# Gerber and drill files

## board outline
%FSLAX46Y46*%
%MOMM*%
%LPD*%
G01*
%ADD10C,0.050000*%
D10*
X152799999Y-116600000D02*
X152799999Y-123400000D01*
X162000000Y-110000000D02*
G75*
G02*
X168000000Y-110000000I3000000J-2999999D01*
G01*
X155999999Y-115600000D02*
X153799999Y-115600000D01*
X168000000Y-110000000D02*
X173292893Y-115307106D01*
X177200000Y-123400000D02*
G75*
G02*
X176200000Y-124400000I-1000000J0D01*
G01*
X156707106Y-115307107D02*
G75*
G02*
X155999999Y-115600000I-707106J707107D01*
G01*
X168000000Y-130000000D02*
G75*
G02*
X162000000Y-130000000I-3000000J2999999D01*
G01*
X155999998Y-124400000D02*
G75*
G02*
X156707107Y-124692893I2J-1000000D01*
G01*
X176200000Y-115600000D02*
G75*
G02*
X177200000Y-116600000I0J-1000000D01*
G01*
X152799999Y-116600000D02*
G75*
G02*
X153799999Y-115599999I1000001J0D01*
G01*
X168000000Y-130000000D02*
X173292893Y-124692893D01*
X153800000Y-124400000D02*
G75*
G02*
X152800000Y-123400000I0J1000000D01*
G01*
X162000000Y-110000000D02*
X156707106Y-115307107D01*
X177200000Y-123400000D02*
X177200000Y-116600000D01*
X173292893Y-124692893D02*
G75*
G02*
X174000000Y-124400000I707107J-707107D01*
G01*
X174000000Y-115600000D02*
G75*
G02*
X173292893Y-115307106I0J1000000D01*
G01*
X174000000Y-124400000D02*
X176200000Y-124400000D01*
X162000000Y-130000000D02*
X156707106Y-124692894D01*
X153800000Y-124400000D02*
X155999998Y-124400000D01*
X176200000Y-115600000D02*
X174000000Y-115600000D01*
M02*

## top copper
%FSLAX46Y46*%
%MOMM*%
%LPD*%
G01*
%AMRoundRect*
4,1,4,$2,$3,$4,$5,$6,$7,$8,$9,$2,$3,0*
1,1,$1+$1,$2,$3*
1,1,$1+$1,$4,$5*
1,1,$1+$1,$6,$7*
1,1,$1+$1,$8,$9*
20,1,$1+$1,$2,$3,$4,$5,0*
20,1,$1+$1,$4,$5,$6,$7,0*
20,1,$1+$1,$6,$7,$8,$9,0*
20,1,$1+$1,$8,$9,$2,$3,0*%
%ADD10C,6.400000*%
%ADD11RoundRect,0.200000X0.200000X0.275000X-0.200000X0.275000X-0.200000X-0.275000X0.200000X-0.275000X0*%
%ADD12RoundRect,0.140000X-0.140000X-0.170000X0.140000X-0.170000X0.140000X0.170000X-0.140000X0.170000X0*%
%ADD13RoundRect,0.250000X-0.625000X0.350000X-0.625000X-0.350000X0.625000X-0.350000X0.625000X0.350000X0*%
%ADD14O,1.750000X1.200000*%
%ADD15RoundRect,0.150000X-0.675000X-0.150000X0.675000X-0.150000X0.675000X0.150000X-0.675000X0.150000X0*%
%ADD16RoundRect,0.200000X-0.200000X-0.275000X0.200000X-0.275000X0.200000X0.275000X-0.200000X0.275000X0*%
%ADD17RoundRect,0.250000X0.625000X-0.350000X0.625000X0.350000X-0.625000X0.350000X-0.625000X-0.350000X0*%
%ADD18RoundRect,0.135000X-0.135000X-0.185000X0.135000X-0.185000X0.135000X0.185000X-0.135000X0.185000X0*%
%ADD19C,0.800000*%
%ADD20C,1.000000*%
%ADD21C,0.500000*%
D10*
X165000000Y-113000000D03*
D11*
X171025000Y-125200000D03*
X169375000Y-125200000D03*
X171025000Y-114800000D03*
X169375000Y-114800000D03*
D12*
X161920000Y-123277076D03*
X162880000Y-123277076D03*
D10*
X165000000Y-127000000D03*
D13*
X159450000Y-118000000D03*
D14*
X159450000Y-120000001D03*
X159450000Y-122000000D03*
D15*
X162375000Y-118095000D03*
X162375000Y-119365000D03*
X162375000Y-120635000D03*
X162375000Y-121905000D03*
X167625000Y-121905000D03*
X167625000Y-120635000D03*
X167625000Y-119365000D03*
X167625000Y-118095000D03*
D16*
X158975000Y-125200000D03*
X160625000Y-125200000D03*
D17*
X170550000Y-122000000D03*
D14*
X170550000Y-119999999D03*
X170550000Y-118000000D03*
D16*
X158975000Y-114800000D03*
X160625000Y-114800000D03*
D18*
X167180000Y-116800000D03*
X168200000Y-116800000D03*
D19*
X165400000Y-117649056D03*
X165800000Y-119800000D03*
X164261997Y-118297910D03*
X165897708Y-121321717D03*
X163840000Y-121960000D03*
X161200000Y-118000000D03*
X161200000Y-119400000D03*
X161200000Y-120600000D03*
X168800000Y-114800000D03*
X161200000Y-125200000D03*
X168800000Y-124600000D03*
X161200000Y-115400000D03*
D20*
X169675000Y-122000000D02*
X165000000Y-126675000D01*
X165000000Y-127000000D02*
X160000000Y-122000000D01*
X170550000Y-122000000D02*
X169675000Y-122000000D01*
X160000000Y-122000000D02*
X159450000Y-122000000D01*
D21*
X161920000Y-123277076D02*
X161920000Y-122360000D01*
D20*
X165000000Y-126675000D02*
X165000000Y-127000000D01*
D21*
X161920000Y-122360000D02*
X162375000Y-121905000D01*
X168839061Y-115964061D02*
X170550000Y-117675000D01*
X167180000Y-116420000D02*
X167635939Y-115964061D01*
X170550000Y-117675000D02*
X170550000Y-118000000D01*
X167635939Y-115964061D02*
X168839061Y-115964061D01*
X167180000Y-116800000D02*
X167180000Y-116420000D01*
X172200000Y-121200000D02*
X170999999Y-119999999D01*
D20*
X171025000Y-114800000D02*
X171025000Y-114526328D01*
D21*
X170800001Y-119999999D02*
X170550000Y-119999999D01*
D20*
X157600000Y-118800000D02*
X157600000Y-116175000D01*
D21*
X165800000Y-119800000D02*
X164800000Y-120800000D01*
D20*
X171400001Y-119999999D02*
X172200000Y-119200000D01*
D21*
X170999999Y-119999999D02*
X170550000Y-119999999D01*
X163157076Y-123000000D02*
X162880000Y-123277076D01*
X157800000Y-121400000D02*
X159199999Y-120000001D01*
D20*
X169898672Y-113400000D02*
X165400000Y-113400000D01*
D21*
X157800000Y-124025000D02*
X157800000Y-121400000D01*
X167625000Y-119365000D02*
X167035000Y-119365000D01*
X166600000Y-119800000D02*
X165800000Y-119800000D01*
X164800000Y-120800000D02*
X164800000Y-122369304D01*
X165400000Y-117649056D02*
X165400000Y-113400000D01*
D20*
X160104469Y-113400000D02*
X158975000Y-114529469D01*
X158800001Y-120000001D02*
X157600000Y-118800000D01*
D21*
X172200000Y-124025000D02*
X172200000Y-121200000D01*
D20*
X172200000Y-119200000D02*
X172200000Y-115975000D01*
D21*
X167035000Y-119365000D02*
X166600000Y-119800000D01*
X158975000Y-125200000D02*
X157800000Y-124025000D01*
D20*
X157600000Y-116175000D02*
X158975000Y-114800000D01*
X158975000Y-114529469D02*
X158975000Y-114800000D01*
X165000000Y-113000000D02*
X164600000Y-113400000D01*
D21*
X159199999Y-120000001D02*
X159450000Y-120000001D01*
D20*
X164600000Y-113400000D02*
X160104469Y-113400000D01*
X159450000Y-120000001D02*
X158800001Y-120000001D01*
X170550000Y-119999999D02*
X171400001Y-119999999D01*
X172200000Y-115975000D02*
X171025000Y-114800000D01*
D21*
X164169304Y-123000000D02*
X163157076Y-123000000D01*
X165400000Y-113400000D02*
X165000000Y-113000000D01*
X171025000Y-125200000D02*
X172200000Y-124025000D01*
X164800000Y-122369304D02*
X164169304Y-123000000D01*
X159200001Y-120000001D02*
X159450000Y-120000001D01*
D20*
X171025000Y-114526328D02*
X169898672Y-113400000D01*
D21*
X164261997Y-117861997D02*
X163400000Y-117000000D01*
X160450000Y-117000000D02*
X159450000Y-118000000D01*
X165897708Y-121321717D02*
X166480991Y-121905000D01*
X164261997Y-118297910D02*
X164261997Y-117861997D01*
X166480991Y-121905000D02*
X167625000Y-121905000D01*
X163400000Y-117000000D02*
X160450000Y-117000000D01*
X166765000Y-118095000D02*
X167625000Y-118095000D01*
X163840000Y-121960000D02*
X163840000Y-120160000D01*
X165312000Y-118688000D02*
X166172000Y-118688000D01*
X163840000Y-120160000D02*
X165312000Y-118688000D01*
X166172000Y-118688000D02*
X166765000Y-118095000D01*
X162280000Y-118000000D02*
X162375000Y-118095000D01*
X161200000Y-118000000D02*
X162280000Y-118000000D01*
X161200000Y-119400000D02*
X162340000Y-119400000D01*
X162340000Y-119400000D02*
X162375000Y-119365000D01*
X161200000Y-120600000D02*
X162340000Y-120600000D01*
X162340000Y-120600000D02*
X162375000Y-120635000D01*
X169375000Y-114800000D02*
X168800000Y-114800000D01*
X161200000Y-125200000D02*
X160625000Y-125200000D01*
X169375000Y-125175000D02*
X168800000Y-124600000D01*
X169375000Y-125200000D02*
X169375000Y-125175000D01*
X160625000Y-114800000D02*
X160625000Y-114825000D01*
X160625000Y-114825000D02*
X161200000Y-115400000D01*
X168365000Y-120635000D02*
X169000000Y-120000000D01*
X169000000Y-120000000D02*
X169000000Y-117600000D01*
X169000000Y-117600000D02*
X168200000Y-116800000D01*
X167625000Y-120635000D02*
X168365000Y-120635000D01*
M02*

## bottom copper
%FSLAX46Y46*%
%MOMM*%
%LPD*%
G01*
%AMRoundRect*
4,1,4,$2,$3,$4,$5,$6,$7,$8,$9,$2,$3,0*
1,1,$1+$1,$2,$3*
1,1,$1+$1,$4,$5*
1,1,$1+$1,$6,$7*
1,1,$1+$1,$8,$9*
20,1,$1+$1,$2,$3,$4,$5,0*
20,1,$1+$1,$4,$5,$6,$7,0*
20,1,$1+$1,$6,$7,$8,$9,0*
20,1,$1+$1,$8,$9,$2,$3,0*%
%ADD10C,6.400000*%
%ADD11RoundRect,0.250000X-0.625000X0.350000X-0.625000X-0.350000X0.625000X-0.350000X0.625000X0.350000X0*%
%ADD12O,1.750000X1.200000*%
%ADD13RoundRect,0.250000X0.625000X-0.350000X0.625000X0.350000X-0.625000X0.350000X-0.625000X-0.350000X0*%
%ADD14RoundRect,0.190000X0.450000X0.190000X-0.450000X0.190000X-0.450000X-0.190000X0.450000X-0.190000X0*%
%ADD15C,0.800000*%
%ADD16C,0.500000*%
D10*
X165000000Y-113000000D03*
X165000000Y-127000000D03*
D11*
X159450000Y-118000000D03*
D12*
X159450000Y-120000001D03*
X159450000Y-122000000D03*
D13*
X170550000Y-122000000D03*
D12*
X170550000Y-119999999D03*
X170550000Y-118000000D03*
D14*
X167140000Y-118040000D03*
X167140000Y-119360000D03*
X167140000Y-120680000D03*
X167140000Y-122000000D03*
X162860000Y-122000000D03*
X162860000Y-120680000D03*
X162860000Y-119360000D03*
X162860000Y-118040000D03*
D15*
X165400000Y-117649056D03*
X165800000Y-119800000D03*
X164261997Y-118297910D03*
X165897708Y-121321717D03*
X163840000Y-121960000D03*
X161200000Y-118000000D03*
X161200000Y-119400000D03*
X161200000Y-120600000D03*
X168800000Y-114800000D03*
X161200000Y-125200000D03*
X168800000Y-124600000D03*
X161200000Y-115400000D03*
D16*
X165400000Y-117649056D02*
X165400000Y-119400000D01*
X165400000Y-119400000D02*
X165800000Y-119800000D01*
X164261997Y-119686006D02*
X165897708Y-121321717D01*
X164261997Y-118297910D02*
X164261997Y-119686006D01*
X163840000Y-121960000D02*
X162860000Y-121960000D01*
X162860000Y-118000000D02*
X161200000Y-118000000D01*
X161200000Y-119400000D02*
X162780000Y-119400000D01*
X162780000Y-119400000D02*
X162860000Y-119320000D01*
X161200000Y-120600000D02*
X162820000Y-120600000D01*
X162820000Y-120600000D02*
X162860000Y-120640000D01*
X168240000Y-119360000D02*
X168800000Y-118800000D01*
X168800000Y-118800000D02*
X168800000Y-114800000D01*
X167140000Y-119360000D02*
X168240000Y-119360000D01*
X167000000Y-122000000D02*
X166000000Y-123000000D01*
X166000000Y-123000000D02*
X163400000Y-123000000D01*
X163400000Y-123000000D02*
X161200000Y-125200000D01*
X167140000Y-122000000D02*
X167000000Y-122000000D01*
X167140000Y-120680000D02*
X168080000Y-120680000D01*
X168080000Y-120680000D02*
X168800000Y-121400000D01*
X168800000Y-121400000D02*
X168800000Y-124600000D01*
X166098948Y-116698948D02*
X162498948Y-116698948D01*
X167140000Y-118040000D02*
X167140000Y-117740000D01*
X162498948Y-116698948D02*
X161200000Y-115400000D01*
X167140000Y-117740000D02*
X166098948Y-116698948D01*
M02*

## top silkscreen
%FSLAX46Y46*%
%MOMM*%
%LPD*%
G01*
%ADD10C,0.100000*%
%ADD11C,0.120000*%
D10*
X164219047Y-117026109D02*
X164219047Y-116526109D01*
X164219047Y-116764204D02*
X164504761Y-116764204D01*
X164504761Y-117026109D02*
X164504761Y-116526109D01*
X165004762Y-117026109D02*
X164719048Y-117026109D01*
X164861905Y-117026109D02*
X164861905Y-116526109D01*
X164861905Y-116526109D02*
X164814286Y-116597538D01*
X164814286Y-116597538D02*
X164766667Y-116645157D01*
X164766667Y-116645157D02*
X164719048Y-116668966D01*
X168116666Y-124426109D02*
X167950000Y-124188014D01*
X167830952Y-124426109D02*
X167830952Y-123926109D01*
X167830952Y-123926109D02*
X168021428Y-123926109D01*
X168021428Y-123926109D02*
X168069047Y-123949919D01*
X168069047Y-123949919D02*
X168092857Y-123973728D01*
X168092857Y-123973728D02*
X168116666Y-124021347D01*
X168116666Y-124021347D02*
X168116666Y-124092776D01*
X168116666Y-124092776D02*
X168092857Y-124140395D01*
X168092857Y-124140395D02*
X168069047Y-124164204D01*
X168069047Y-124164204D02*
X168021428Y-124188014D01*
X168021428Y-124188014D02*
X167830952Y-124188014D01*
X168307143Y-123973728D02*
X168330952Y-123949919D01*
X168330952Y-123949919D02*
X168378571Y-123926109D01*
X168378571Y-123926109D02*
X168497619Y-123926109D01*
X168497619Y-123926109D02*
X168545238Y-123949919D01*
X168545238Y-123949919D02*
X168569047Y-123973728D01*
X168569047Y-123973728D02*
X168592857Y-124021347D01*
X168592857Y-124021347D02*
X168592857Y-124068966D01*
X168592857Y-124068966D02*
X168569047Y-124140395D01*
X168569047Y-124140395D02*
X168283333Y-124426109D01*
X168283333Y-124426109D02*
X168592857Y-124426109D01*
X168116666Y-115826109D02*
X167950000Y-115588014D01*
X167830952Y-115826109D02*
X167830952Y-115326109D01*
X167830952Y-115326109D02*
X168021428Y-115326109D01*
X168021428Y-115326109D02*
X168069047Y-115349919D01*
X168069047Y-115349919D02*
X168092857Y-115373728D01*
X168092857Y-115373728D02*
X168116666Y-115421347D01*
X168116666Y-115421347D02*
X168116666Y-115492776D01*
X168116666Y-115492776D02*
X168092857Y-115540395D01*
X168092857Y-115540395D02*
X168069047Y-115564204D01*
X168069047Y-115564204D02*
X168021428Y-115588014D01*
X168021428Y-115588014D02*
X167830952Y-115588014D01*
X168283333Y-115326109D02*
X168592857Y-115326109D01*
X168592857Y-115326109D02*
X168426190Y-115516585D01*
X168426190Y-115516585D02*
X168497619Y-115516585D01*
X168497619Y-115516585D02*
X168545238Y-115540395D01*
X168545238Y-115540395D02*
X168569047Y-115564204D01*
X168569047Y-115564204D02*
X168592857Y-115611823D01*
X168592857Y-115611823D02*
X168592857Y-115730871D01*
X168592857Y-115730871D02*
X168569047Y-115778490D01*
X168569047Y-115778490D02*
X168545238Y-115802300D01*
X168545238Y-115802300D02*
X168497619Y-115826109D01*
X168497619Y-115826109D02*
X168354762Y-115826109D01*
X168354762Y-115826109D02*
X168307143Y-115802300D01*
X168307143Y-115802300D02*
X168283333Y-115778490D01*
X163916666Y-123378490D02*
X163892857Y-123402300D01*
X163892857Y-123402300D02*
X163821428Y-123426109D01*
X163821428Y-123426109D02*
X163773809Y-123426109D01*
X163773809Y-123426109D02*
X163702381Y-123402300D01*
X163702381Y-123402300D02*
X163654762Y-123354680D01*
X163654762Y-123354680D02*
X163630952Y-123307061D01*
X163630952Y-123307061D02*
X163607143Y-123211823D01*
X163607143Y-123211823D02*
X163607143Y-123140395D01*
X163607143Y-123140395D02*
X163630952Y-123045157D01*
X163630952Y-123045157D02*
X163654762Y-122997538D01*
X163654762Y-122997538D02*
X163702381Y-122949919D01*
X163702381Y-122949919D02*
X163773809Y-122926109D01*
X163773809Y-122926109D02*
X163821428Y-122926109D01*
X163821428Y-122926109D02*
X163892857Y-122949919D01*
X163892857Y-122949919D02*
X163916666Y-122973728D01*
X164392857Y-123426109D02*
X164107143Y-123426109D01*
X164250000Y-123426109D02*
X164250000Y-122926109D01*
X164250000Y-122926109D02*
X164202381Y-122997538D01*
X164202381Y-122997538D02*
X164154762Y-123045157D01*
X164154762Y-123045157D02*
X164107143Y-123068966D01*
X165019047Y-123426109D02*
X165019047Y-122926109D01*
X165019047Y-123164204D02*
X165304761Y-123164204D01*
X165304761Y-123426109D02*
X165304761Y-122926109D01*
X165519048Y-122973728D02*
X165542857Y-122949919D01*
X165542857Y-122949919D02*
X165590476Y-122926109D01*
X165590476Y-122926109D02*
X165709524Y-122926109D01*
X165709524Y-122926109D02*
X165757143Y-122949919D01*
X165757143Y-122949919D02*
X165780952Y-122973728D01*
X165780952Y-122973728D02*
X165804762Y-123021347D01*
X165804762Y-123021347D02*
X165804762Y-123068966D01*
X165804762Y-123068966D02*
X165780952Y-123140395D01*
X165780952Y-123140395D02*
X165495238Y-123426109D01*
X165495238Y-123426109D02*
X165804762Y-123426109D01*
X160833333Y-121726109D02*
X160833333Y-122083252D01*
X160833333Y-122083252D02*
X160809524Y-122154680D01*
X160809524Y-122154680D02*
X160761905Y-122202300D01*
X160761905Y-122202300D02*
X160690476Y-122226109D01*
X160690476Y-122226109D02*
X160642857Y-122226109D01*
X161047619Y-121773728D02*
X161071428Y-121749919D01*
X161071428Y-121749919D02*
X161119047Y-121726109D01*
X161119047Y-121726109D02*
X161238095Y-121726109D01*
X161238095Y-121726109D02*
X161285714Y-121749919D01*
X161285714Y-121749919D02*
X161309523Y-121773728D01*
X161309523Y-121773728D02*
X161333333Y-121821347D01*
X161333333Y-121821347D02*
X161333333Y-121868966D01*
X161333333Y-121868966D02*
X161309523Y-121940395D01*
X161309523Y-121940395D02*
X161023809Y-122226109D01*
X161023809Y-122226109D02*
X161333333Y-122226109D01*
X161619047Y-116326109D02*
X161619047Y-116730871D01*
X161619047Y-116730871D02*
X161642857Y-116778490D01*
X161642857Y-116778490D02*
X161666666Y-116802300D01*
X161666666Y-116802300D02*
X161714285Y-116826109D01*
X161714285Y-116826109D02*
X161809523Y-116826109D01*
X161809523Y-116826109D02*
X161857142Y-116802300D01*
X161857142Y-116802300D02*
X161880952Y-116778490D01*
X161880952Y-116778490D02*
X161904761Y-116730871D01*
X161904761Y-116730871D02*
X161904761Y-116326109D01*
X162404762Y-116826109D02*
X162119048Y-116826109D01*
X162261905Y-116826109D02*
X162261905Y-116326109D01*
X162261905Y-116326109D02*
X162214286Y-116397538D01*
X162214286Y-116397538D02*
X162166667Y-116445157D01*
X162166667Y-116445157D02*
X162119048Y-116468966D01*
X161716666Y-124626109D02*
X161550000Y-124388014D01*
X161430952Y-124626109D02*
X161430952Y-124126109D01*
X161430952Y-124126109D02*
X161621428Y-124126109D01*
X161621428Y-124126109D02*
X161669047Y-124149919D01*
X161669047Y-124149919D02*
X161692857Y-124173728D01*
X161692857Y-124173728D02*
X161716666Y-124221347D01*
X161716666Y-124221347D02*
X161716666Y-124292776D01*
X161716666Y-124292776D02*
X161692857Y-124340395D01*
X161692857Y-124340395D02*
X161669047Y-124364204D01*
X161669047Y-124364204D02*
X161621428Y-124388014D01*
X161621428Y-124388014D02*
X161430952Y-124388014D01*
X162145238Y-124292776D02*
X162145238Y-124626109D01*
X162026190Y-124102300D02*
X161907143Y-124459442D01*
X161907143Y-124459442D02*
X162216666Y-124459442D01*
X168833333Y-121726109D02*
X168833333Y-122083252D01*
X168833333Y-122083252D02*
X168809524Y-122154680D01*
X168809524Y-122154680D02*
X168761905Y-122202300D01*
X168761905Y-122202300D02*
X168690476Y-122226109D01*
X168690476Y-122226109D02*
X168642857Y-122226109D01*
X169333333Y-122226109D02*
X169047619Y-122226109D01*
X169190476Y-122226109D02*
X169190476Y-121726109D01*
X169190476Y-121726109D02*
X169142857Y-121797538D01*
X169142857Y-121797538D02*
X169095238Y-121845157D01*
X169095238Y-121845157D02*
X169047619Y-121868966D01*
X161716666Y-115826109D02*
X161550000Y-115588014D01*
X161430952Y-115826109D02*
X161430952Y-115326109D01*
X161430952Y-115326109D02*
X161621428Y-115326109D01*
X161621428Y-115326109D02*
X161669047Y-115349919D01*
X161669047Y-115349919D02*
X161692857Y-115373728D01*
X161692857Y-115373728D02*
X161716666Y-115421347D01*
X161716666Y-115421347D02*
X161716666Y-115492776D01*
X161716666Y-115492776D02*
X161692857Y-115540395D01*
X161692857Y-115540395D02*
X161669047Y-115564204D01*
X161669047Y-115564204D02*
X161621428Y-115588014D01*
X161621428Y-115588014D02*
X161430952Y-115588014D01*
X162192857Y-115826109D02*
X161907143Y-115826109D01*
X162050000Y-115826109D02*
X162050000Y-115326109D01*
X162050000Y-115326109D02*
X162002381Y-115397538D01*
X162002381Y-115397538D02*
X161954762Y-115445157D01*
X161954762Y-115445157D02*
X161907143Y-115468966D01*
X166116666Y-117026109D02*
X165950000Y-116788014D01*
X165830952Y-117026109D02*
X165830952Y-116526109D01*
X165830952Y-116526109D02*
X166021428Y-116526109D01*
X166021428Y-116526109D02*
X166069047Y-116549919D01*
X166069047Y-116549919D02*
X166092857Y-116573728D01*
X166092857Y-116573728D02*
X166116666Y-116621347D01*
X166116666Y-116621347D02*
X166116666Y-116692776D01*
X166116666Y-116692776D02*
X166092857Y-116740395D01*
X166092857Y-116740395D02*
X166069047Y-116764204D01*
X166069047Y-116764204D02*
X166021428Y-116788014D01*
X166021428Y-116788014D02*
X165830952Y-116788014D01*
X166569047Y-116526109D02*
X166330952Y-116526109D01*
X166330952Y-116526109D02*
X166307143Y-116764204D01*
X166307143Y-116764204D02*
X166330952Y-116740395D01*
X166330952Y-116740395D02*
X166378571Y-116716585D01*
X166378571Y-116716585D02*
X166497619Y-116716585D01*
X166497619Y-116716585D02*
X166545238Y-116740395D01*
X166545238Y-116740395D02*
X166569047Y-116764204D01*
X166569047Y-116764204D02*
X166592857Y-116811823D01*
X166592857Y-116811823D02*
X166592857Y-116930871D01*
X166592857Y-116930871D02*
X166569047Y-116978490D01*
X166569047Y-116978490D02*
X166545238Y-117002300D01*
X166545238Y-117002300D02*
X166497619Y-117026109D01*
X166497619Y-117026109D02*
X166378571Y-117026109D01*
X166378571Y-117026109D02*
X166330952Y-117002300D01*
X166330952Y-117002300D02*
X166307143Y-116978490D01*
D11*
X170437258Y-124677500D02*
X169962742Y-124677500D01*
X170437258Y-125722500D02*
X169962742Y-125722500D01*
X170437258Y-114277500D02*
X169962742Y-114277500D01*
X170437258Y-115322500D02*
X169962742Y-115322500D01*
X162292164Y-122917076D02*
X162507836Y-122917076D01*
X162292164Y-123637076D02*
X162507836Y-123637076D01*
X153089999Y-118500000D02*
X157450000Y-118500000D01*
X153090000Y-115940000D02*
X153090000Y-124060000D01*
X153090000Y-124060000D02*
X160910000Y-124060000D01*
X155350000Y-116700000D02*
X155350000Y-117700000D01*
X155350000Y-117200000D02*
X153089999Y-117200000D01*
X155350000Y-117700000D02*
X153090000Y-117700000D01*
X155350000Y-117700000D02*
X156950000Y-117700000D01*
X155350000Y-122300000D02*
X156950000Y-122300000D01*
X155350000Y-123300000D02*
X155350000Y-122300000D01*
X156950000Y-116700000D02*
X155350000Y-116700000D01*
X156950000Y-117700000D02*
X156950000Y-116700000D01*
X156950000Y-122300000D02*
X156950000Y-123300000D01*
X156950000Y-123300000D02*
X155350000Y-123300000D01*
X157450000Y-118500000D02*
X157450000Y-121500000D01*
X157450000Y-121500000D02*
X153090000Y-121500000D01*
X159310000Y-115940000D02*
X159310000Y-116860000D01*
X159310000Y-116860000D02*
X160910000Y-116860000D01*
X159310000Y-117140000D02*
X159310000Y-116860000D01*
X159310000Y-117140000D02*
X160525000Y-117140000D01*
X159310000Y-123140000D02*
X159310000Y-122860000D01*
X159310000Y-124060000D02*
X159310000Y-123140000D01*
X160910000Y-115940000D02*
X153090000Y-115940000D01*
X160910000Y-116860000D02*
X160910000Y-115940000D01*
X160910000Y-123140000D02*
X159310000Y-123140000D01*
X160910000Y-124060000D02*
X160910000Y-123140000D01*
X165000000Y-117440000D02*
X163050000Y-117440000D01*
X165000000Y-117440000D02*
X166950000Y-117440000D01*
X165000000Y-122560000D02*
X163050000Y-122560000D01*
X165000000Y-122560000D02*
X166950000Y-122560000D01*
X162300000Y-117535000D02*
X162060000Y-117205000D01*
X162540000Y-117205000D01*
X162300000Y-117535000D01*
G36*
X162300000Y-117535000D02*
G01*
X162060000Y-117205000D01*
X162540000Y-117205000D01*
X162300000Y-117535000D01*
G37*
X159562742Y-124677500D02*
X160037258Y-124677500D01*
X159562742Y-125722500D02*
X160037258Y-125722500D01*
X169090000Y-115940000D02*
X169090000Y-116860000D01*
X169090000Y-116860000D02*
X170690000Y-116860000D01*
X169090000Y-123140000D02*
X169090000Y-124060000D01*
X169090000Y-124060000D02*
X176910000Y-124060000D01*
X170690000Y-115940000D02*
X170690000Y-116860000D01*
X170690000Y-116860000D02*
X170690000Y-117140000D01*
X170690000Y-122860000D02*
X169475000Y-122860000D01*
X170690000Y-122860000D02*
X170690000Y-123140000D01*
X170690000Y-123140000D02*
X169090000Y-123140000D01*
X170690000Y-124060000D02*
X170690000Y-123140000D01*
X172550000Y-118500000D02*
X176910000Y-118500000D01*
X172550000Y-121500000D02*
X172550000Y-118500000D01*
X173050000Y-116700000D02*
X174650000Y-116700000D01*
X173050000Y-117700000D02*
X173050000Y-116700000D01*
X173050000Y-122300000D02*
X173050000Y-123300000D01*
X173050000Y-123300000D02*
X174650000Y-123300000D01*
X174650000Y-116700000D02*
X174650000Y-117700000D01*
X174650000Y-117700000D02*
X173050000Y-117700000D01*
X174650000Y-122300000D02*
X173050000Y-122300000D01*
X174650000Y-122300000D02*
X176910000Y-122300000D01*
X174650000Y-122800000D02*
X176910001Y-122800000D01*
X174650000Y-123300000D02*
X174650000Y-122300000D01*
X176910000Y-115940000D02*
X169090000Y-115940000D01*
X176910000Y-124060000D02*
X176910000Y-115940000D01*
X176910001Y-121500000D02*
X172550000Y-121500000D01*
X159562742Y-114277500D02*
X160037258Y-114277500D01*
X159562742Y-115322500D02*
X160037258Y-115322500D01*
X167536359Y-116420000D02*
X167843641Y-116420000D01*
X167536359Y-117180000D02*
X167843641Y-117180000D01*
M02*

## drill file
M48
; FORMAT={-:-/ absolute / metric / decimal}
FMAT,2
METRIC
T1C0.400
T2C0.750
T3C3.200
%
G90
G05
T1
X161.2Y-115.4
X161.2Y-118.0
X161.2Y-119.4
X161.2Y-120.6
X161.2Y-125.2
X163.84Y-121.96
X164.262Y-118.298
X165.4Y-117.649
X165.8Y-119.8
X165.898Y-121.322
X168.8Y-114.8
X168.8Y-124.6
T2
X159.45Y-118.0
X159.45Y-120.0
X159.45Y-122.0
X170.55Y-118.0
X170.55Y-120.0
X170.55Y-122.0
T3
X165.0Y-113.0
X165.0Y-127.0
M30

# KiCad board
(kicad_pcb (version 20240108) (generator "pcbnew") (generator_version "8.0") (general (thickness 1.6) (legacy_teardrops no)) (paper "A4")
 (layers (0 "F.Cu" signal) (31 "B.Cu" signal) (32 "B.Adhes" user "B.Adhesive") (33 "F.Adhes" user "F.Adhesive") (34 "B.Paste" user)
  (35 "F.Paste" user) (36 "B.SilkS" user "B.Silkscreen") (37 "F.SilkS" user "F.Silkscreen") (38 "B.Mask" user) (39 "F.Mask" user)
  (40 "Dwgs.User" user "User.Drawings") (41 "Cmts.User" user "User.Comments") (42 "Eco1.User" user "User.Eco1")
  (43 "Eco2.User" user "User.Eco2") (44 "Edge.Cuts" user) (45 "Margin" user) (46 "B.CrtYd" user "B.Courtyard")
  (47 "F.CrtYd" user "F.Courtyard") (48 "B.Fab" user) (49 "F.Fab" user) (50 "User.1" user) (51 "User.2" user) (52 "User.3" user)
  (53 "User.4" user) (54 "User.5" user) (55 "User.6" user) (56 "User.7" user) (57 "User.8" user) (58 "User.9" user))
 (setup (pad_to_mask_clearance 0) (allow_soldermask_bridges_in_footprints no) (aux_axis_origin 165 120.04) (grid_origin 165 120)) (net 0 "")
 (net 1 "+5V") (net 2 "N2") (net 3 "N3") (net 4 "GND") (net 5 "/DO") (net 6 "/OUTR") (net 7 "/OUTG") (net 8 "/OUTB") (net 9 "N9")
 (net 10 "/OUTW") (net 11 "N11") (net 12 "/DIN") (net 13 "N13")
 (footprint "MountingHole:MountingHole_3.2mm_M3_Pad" (layer "F.Cu") (at 165 113)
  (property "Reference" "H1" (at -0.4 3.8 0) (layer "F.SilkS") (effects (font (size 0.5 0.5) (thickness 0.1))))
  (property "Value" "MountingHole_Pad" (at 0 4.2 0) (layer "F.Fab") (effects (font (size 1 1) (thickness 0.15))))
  (pad "1" thru_hole circle (at 0 0) (size 6.4 6.4) (drill 3.2) (layers "*.Cu" "*.Mask") (remove_unused_layers no) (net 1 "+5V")))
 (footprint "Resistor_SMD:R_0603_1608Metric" (layer "F.Cu") (at 170.2 125.2 180)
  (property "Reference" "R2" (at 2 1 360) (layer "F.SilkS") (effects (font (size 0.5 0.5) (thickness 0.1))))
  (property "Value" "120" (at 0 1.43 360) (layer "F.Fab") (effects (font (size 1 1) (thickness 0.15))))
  (fp_line (start -0.237258 0.5225) (end 0.237258 0.5225) (stroke (width 0.12) (type solid)) (layer "F.SilkS"))
  (fp_line (start -0.237258 -0.5225) (end 0.237258 -0.5225) (stroke (width 0.12) (type solid)) (layer "F.SilkS"))
  (pad "1" smd roundrect (at -0.825 0 180) (size 0.8 0.95) (layers "F.Cu" "F.Paste" "F.Mask") (roundrect_rratio 0.25) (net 1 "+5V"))
  (pad "2" smd roundrect (at 0.825 0 180) (size 0.8 0.95) (layers "F.Cu" "F.Paste" "F.Mask") (roundrect_rratio 0.25) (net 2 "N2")))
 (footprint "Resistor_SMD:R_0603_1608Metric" (layer "F.Cu") (at 170.2 114.8 180)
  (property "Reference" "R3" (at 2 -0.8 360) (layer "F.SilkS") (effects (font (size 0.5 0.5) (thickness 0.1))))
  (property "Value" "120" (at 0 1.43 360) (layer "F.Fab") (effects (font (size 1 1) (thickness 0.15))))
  (fp_line (start -0.237258 0.5225) (end 0.237258 0.5225) (stroke (width 0.12) (type solid)) (layer "F.SilkS"))
  (fp_line (start -0.237258 -0.5225) (end 0.237258 -0.5225) (stroke (width 0.12) (type solid)) (layer "F.SilkS"))
  (pad "1" smd roundrect (at -0.825 0 180) (size 0.8 0.95) (layers "F.Cu" "F.Paste" "F.Mask") (roundrect_rratio 0.25) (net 1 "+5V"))
  (pad "2" smd roundrect (at 0.825 0 180) (size 0.8 0.95) (layers "F.Cu" "F.Paste" "F.Mask") (roundrect_rratio 0.25) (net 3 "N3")))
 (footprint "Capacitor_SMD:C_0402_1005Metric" (layer "F.Cu") (at 162.4 123.277076)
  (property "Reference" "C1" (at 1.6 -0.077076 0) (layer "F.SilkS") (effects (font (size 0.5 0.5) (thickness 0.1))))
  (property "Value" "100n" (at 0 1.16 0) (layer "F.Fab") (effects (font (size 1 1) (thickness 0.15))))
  (fp_line (start -0.107836 -0.36) (end 0.107836 -0.36) (stroke (width 0.12) (type solid)) (layer "F.SilkS"))
  (fp_line (start -0.107836 0.36) (end 0.107836 0.36) (stroke (width 0.12) (type solid)) (layer "F.SilkS"))
  (pad "1" smd roundrect (at -0.48 0) (size 0.56 0.62) (layers "F.Cu" "F.Paste" "F.Mask") (roundrect_rratio 0.25) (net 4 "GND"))
  (pad "2" smd roundrect (at 0.48 0) (size 0.56 0.62) (layers "F.Cu" "F.Paste" "F.Mask") (roundrect_rratio 0.25) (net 1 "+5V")))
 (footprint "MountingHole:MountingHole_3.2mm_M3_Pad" (layer "F.Cu") (at 165 127)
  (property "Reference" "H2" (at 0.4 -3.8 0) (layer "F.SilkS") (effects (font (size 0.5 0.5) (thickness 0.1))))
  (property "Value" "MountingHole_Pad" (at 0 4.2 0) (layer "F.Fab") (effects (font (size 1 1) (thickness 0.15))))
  (pad "1" thru_hole circle (at 0 0) (size 6.4 6.4) (drill 3.2) (layers "*.Cu" "*.Mask") (remove_unused_layers no) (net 4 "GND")))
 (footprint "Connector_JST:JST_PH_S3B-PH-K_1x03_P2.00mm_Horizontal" (layer "F.Cu") (at 159.45 118 -90)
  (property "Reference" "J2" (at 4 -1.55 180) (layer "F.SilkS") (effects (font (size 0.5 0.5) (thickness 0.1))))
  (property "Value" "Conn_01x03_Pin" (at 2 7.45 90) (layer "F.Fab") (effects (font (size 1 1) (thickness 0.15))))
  (fp_line (start 0.5 6.360001) (end 0.5 2) (stroke (width 0.12) (type solid)) (layer "F.SilkS"))
  (fp_line (start -2.06 6.36) (end 6.06 6.36) (stroke (width 0.12) (type solid)) (layer "F.SilkS"))
  (fp_line (start 6.06 6.36) (end 6.06 -1.46) (stroke (width 0.12) (type solid)) (layer "F.SilkS"))
  (fp_line (start -1.3 4.1) (end -0.3 4.1) (stroke (width 0.12) (type solid)) (layer "F.SilkS"))
  (fp_line (start -0.8 4.1) (end -0.8 6.360001) (stroke (width 0.12) (type solid)) (layer "F.SilkS"))
  (fp_line (start -0.3 4.1) (end -0.3 6.36) (stroke (width 0.12) (type solid)) (layer "F.SilkS"))
  (fp_line (start -0.3 4.1) (end -0.3 2.5) (stroke (width 0.12) (type solid)) (layer "F.SilkS"))
  (fp_line (start 4.3 4.1) (end 4.3 2.5) (stroke (width 0.12) (type solid)) (layer "F.SilkS"))
  (fp_line (start 5.3 4.1) (end 4.3 4.1) (stroke (width 0.12) (type solid)) (layer "F.SilkS"))
  (fp_line (start -1.3 2.5) (end -1.3 4.1) (stroke (width 0.12) (type solid)) (layer "F.SilkS"))
  (fp_line (start -0.3 2.5) (end -1.3 2.5) (stroke (width 0.12) (type solid)) (layer "F.SilkS"))
  (fp_line (start 4.3 2.5) (end 5.3 2.5) (stroke (width 0.12) (type solid)) (layer "F.SilkS"))
  (fp_line (start 5.3 2.5) (end 5.3 4.1) (stroke (width 0.12) (type solid)) (layer "F.SilkS"))
  (fp_line (start 0.5 2) (end 3.5 2) (stroke (width 0.12) (type solid)) (layer "F.SilkS"))
  (fp_line (start 3.5 2) (end 3.5 6.36) (stroke (width 0.12) (type solid)) (layer "F.SilkS"))
  (fp_line (start -2.06 0.14) (end -1.14 0.14) (stroke (width 0.12) (type solid)) (layer "F.SilkS"))
  (fp_line (start -1.14 0.14) (end -1.14 -1.46) (stroke (width 0.12) (type solid)) (layer "F.SilkS"))
  (fp_line (start -0.86 0.14) (end -1.14 0.14) (stroke (width 0.12) (type solid)) (layer "F.SilkS"))
  (fp_line (start -0.86 0.14) (end -0.86 -1.075) (stroke (width 0.12) (type solid)) (layer "F.SilkS"))
  (fp_line (start 5.14 0.14) (end 4.86 0.14) (stroke (width 0.12) (type solid)) (layer "F.SilkS"))
  (fp_line (start 6.06 0.14) (end 5.14 0.14) (stroke (width 0.12) (type solid)) (layer "F.SilkS"))
  (fp_line (start -2.06 -1.46) (end -2.06 6.36) (stroke (width 0.12) (type solid)) (layer "F.SilkS"))
  (fp_line (start -1.14 -1.46) (end -2.06 -1.46) (stroke (width 0.12) (type solid)) (layer "F.SilkS"))
  (fp_line (start 5.14 -1.46) (end 5.14 0.14) (stroke (width 0.12) (type solid)) (layer "F.SilkS"))
  (fp_line (start 6.06 -1.46) (end 5.14 -1.46) (stroke (width 0.12) (type solid)) (layer "F.SilkS"))
  (pad "1" thru_hole roundrect (at 0 0 270) (size 1.2 1.75) (drill 0.75) (layers "*.Cu" "*.Mask") (remove_unused_layers no)
   (roundrect_rratio 0.208333) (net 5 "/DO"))
  (pad "2" thru_hole oval (at 2.000001 0 270) (size 1.2 1.75) (drill 0.75) (layers "*.Cu" "*.Mask") (remove_unused_layers no) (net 1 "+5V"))
  (pad "3" thru_hole oval (at 4 0 270) (size 1.2 1.75) (drill 0.75) (layers "*.Cu" "*.Mask") (remove_unused_layers no) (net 4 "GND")))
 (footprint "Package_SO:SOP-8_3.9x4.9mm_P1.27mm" (layer "F.Cu") (at 165 120)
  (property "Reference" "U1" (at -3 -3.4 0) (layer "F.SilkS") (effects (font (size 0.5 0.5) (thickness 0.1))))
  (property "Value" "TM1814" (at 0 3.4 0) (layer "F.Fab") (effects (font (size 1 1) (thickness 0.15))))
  (fp_line (start 0 -2.56) (end -1.95 -2.56) (stroke (width 0.12) (type solid)) (layer "F.SilkS"))
  (fp_line (start 0 -2.56) (end 1.95 -2.56) (stroke (width 0.12) (type solid)) (layer "F.SilkS"))
  (fp_line (start 0 2.56) (end -1.95 2.56) (stroke (width 0.12) (type solid)) (layer "F.SilkS"))
  (fp_line (start 0 2.56) (end 1.95 2.56) (stroke (width 0.12) (type solid)) (layer "F.SilkS"))
  (fp_poly
   (pts (xy -2.7 -2.465) (xy -2.94 -2.795) (xy -2.46 -2.795) (xy -2.7 -2.465)) (stroke (width 0.12) (type solid)) (fill solid)
   (layer "F.SilkS"))
  (pad "1" smd roundrect (at -2.625 -1.905) (size 1.65 0.6) (layers "F.Cu" "F.Paste" "F.Mask") (roundrect_rratio 0.25) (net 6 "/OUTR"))
  (pad "2" smd roundrect (at -2.625 -0.635) (size 1.65 0.6) (layers "F.Cu" "F.Paste" "F.Mask") (roundrect_rratio 0.25) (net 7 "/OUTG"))
  (pad "3" smd roundrect (at -2.625 0.635) (size 1.65 0.6) (layers "F.Cu" "F.Paste" "F.Mask") (roundrect_rratio 0.25) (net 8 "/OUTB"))
  (pad "4" smd roundrect (at -2.625 1.905) (size 1.65 0.6) (layers "F.Cu" "F.Paste" "F.Mask") (roundrect_rratio 0.25) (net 4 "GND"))
  (pad "5" smd roundrect (at 2.625 1.905) (size 1.65 0.6) (layers "F.Cu" "F.Paste" "F.Mask") (roundrect_rratio 0.25) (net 5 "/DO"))
  (pad "6" smd roundrect (at 2.625 0.635) (size 1.65 0.6) (layers "F.Cu" "F.Paste" "F.Mask") (roundrect_rratio 0.25) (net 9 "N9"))
  (pad "7" smd roundrect (at 2.625 -0.635) (size 1.65 0.6) (layers "F.Cu" "F.Paste" "F.Mask") (roundrect_rratio 0.25) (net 1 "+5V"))
  (pad "8" smd roundrect (at 2.625 -1.905) (size 1.65 0.6) (layers "F.Cu" "F.Paste" "F.Mask") (roundrect_rratio 0.25) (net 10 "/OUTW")))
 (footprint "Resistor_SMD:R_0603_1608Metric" (layer "F.Cu") (at 159.8 125.2)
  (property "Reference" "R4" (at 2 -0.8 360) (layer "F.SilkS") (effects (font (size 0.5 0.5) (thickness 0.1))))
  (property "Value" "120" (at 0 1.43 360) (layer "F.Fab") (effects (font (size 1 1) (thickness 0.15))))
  (fp_line (start -0.237258 -0.5225) (end 0.237258 -0.5225) (stroke (width 0.12) (type solid)) (layer "F.SilkS"))
  (fp_line (start -0.237258 0.5225) (end 0.237258 0.5225) (stroke (width 0.12) (type solid)) (layer "F.SilkS"))
  (pad "1" smd roundrect (at -0.825 0) (size 0.8 0.95) (layers "F.Cu" "F.Paste" "F.Mask") (roundrect_rratio 0.25) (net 1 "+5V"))
  (pad "2" smd roundrect (at 0.825 0) (size 0.8 0.95) (layers "F.Cu" "F.Paste" "F.Mask") (roundrect_rratio 0.25) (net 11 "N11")))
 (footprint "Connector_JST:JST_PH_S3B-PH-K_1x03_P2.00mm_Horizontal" (layer "F.Cu") (at 170.55 122 90)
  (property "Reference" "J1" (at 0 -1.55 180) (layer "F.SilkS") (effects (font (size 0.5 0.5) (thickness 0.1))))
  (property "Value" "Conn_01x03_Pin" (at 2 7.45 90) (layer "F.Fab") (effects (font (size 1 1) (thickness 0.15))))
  (fp_line (start 6.06 -1.46) (end 5.14 -1.46) (stroke (width 0.12) (type solid)) (layer "F.SilkS"))
  (fp_line (start 5.14 -1.46) (end 5.14 0.14) (stroke (width 0.12) (type solid)) (layer "F.SilkS"))
  (fp_line (start -1.14 -1.46) (end -2.06 -1.46) (stroke (width 0.12) (type solid)) (layer "F.SilkS"))
  (fp_line (start -2.06 -1.46) (end -2.06 6.36) (stroke (width 0.12) (type solid)) (layer "F.SilkS"))
  (fp_line (start 6.06 0.14) (end 5.14 0.14) (stroke (width 0.12) (type solid)) (layer "F.SilkS"))
  (fp_line (start 5.14 0.14) (end 4.86 0.14) (stroke (width 0.12) (type solid)) (layer "F.SilkS"))
  (fp_line (start -0.86 0.14) (end -0.86 -1.075) (stroke (width 0.12) (type solid)) (layer "F.SilkS"))
  (fp_line (start -0.86 0.14) (end -1.14 0.14) (stroke (width 0.12) (type solid)) (layer "F.SilkS"))
  (fp_line (start -1.14 0.14) (end -1.14 -1.46) (stroke (width 0.12) (type solid)) (layer "F.SilkS"))
  (fp_line (start -2.06 0.14) (end -1.14 0.14) (stroke (width 0.12) (type solid)) (layer "F.SilkS"))
  (fp_line (start 3.5 2) (end 3.5 6.36) (stroke (width 0.12) (type solid)) (layer "F.SilkS"))
  (fp_line (start 0.5 2) (end 3.5 2) (stroke (width 0.12) (type solid)) (layer "F.SilkS"))
  (fp_line (start 5.3 2.5) (end 5.3 4.1) (stroke (width 0.12) (type solid)) (layer "F.SilkS"))
  (fp_line (start 4.3 2.5) (end 5.3 2.5) (stroke (width 0.12) (type solid)) (layer "F.SilkS"))
  (fp_line (start -0.3 2.5) (end -1.3 2.5) (stroke (width 0.12) (type solid)) (layer "F.SilkS"))
  (fp_line (start -1.3 2.5) (end -1.3 4.1) (stroke (width 0.12) (type solid)) (layer "F.SilkS"))
  (fp_line (start 5.3 4.1) (end 4.3 4.1) (stroke (width 0.12) (type solid)) (layer "F.SilkS"))
  (fp_line (start 4.3 4.1) (end 4.3 2.5) (stroke (width 0.12) (type solid)) (layer "F.SilkS"))
  (fp_line (start -0.3 4.1) (end -0.3 2.5) (stroke (width 0.12) (type solid)) (layer "F.SilkS"))
  (fp_line (start -0.3 4.1) (end -0.3 6.36) (stroke (width 0.12) (type solid)) (layer "F.SilkS"))
  (fp_line (start -0.8 4.1) (end -0.8 6.360001) (stroke (width 0.12) (type solid)) (layer "F.SilkS"))
  (fp_line (start -1.3 4.1) (end -0.3 4.1) (stroke (width 0.12) (type solid)) (layer "F.SilkS"))
  (fp_line (start 6.06 6.36) (end 6.06 -1.46) (stroke (width 0.12) (type solid)) (layer "F.SilkS"))
  (fp_line (start -2.06 6.36) (end 6.06 6.36) (stroke (width 0.12) (type solid)) (layer "F.SilkS"))
  (fp_line (start 0.5 6.360001) (end 0.5 2) (stroke (width 0.12) (type solid)) (layer "F.SilkS"))
  (pad "1" thru_hole roundrect (at 0 0 90) (size 1.2 1.75) (drill 0.75) (layers "*.Cu" "*.Mask") (remove_unused_layers no)
   (roundrect_rratio 0.208333) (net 4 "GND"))
  (pad "2" thru_hole oval (at 2.000001 0 90) (size 1.2 1.75) (drill 0.75) (layers "*.Cu" "*.Mask") (remove_unused_layers no) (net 1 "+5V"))
  (pad "3" thru_hole oval (at 4 0 90) (size 1.2 1.75) (drill 0.75) (layers "*.Cu" "*.Mask") (remove_unused_layers no) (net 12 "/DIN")))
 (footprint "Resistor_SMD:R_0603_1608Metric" (layer "F.Cu") (at 159.8 114.8)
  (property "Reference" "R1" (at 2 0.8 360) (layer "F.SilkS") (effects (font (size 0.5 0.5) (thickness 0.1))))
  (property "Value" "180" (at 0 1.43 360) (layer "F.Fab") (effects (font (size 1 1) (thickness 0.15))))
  (fp_line (start -0.237258 -0.5225) (end 0.237258 -0.5225) (stroke (width 0.12) (type solid)) (layer "F.SilkS"))
  (fp_line (start -0.237258 0.5225) (end 0.237258 0.5225) (stroke (width 0.12) (type solid)) (layer "F.SilkS"))
  (pad "1" smd roundrect (at -0.825 0) (size 0.8 0.95) (layers "F.Cu" "F.Paste" "F.Mask") (roundrect_rratio 0.25) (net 1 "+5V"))
  (pad "2" smd roundrect (at 0.825 0) (size 0.8 0.95) (layers "F.Cu" "F.Paste" "F.Mask") (roundrect_rratio 0.25) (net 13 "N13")))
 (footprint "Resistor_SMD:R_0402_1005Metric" (layer "F.Cu") (at 167.69 116.8)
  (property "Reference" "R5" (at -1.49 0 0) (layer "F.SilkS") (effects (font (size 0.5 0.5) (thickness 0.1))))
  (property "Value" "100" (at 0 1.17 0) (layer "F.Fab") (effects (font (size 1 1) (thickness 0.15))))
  (fp_line (start -0.153641 -0.38) (end 0.153641 -0.38) (stroke (width 0.12) (type solid)) (layer "F.SilkS"))
  (fp_line (start -0.153641 0.38) (end 0.153641 0.38) (stroke (width 0.12) (type solid)) (layer "F.SilkS"))
  (pad "1" smd roundrect (at -0.51 0) (size 0.54 0.64) (layers "F.Cu" "F.Paste" "F.Mask") (roundrect_rratio 0.25) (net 12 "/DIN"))
  (pad "2" smd roundrect (at 0.51 0) (size 0.54 0.64) (layers "F.Cu" "F.Paste" "F.Mask") (roundrect_rratio 0.25) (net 9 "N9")))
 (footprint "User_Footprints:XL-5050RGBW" (layer "B.Cu") (at 165 120.04 180)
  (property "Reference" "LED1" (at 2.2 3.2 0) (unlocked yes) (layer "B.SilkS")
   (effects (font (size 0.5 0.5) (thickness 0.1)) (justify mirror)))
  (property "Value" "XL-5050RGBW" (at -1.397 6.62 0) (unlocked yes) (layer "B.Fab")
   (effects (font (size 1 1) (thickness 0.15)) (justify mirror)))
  (pad "1" smd roundrect (at -2.14 2 180) (size 1.28 0.76) (layers "B.Cu" "B.Paste" "B.Mask") (roundrect_rratio 0.25) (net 13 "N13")
   (thermal_bridge_angle 45))
  (pad "2" smd roundrect (at -2.14 0.68 180) (size 1.28 0.76) (layers "B.Cu" "B.Paste" "B.Mask") (roundrect_rratio 0.25) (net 3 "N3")
   (thermal_bridge_angle 45))
  (pad "3" smd roundrect (at -2.14 -0.64 180) (size 1.28 0.76) (layers "B.Cu" "B.Paste" "B.Mask") (roundrect_rratio 0.25) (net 2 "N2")
   (thermal_bridge_angle 45))
  (pad "4" smd roundrect (at -2.14 -1.96 180) (size 1.28 0.76) (layers "B.Cu" "B.Paste" "B.Mask") (roundrect_rratio 0.25) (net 11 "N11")
   (thermal_bridge_angle 45))
  (pad "5" smd roundrect (at 2.14 -1.96 180) (size 1.28 0.76) (layers "B.Cu" "B.Paste" "B.Mask") (roundrect_rratio 0.25) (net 10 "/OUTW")
   (thermal_bridge_angle 45))
  (pad "6" smd roundrect (at 2.14 -0.64 180) (size 1.28 0.76) (layers "B.Cu" "B.Paste" "B.Mask") (roundrect_rratio 0.25) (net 8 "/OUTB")
   (thermal_bridge_angle 45))
  (pad "7" smd roundrect (at 2.14 0.68 180) (size 1.28 0.76) (layers "B.Cu" "B.Paste" "B.Mask") (roundrect_rratio 0.25) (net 7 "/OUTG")
   (thermal_bridge_angle 45))
  (pad "8" smd roundrect (at 2.14 2 180) (size 1.28 0.76) (layers "B.Cu" "B.Paste" "B.Mask") (roundrect_rratio 0.25) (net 6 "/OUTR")
   (thermal_bridge_angle 45)))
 (gr_line (start 152.799999 116.6) (end 152.799999 123.4) (stroke (width 0.05) (type default)) (layer "Edge.Cuts"))
 (gr_arc (start 162 110) (mid 165 108.757359) (end 168 110) (stroke (width 0.05) (type default)) (layer "Edge.Cuts"))
 (gr_line (start 155.999999 115.6) (end 153.799999 115.6) (stroke (width 0.05) (type default)) (layer "Edge.Cuts"))
 (gr_line (start 168 110) (end 173.292893 115.307106) (stroke (width 0.05) (type default)) (layer "Edge.Cuts"))
 (gr_arc (start 177.2 123.4) (mid 176.907107 124.107107) (end 176.2 124.4) (stroke (width 0.05) (type default)) (layer "Edge.Cuts"))
 (gr_arc (start 156.707106 115.307107) (mid 156.382683 115.52388) (end 155.999999 115.6) (stroke (width 0.05) (type default))
  (layer "Edge.Cuts"))
 (gr_arc (start 168 130) (mid 165 131.242641) (end 162 130) (stroke (width 0.05) (type default)) (layer "Edge.Cuts"))
 (gr_arc (start 155.999998 124.4) (mid 156.382683 124.47612) (end 156.707106 124.692894) (stroke (width 0.05) (type default))
  (layer "Edge.Cuts"))
 (gr_arc (start 176.2 115.6) (mid 176.907107 115.892893) (end 177.2 116.6) (stroke (width 0.05) (type default)) (layer "Edge.Cuts"))
 (gr_arc (start 152.799999 116.6) (mid 153.092893 115.892894) (end 153.799999 115.6) (stroke (width 0.05) (type default))
  (layer "Edge.Cuts"))
 (gr_line (start 168 130) (end 173.292893 124.692893) (stroke (width 0.05) (type default)) (layer "Edge.Cuts"))
 (gr_arc (start 153.8 124.4) (mid 153.092893 124.107107) (end 152.799999 123.4) (stroke (width 0.05) (type default)) (layer "Edge.Cuts"))
 (gr_line (start 162 110) (end 156.707106 115.307107) (stroke (width 0.05) (type default)) (layer "Edge.Cuts"))
 (gr_line (start 177.2 123.4) (end 177.2 116.6) (stroke (width 0.05) (type default)) (layer "Edge.Cuts"))
 (gr_arc (start 173.292893 124.692893) (mid 173.617316 124.47612) (end 174 124.4) (stroke (width 0.05) (type default)) (layer "Edge.Cuts"))
 (gr_arc (start 174 115.6) (mid 173.617316 115.52388) (end 173.292893 115.307106) (stroke (width 0.05) (type default)) (layer "Edge.Cuts"))
 (gr_line (start 174 124.4) (end 176.2 124.4) (stroke (width 0.05) (type default)) (layer "Edge.Cuts"))
 (gr_line (start 162 130) (end 156.707106 124.692894) (stroke (width 0.05) (type default)) (layer "Edge.Cuts"))
 (gr_line (start 153.8 124.4) (end 155.999998 124.4) (stroke (width 0.05) (type default)) (layer "Edge.Cuts"))
 (gr_line (start 176.2 115.6) (end 174 115.6) (stroke (width 0.05) (type default)) (layer "Edge.Cuts"))
 (segment (start 169.675 122) (end 165 126.675) (width 1) (layer "F.Cu") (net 4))
 (segment (start 165 127) (end 160 122) (width 1) (layer "F.Cu") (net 4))
 (segment (start 170.55 122) (end 169.675 122) (width 1) (layer "F.Cu") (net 4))
 (segment (start 160 122) (end 159.45 122) (width 1) (layer "F.Cu") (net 4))
 (segment (start 161.92 123.277076) (end 161.92 122.36) (width 0.5) (layer "F.Cu") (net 4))
 (segment (start 165 126.675) (end 165 127) (width 1) (layer "F.Cu") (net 4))
 (segment (start 161.92 122.36) (end 162.375 121.905) (width 0.5) (layer "F.Cu") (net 4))
 (segment (start 168.839061 115.964061) (end 170.55 117.675) (width 0.5) (layer "F.Cu") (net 12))
 (segment (start 167.18 116.42) (end 167.635939 115.964061) (width 0.5) (layer "F.Cu") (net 12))
 (segment (start 170.55 117.675) (end 170.55 118) (width 0.5) (layer "F.Cu") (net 12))
 (segment (start 167.635939 115.964061) (end 168.839061 115.964061) (width 0.5) (layer "F.Cu") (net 12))
 (segment (start 167.18 116.8) (end 167.18 116.42) (width 0.5) (layer "F.Cu") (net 12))
 (segment (start 172.2 121.2) (end 170.999999 119.999999) (width 0.5) (layer "F.Cu") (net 1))
 (segment (start 171.025 114.8) (end 171.025 114.526328) (width 1) (layer "F.Cu") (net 1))
 (segment (start 170.800001 119.999999) (end 170.55 119.999999) (width 0.5) (layer "F.Cu") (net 1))
 (segment (start 157.6 118.8) (end 157.6 116.175) (width 1) (layer "F.Cu") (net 1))
 (segment (start 165.8 119.8) (end 164.8 120.8) (width 0.5) (layer "F.Cu") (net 1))
 (segment (start 171.400001 119.999999) (end 172.2 119.2) (width 1) (layer "F.Cu") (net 1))
 (segment (start 170.999999 119.999999) (end 170.55 119.999999) (width 0.5) (layer "F.Cu") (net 1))
 (segment (start 163.157076 123) (end 162.88 123.277076) (width 0.5) (layer "F.Cu") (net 1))
 (segment (start 157.8 121.4) (end 159.199999 120.000001) (width 0.5) (layer "F.Cu") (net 1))
 (segment (start 169.898672 113.4) (end 165.4 113.4) (width 1) (layer "F.Cu") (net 1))
 (segment (start 157.8 124.025) (end 157.8 121.4) (width 0.5) (layer "F.Cu") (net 1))
 (segment (start 167.625 119.365) (end 167.035 119.365) (width 0.5) (layer "F.Cu") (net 1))
 (segment (start 166.6 119.8) (end 165.8 119.8) (width 0.5) (layer "F.Cu") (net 1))
 (segment (start 164.8 120.8) (end 164.8 122.369304) (width 0.5) (layer "F.Cu") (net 1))
 (segment (start 165.4 117.649056) (end 165.4 113.4) (width 0.5) (layer "F.Cu") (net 1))
 (segment (start 160.104469 113.4) (end 158.975 114.529469) (width 1) (layer "F.Cu") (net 1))
 (segment (start 158.800001 120.000001) (end 157.6 118.8) (width 1) (layer "F.Cu") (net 1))
 (segment (start 172.2 124.025) (end 172.2 121.2) (width 0.5) (layer "F.Cu") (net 1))
 (segment (start 172.2 119.2) (end 172.2 115.975) (width 1) (layer "F.Cu") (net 1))
 (segment (start 167.035 119.365) (end 166.6 119.8) (width 0.5) (layer "F.Cu") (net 1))
 (segment (start 158.975 125.2) (end 157.8 124.025) (width 0.5) (layer "F.Cu") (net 1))
 (segment (start 157.6 116.175) (end 158.975 114.8) (width 1) (layer "F.Cu") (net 1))
 (segment (start 158.975 114.529469) (end 158.975 114.8) (width 1) (layer "F.Cu") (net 1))
 (segment (start 165 113) (end 164.6 113.4) (width 1) (layer "F.Cu") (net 1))
 (segment (start 159.199999 120.000001) (end 159.45 120.000001) (width 0.5) (layer "F.Cu") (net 1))
 (segment (start 164.6 113.4) (end 160.104469 113.4) (width 1) (layer "F.Cu") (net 1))
 (segment (start 159.45 120.000001) (end 158.800001 120.000001) (width 1) (layer "F.Cu") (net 1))
 (segment (start 170.55 119.999999) (end 171.400001 119.999999) (width 1) (layer "F.Cu") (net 1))
 (segment (start 172.2 115.975) (end 171.025 114.8) (width 1) (layer "F.Cu") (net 1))
 (segment (start 164.169304 123) (end 163.157076 123) (width 0.5) (layer "F.Cu") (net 1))
 (segment (start 165.4 113.4) (end 165 113) (width 0.5) (layer "F.Cu") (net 1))
 (segment (start 171.025 125.2) (end 172.2 124.025) (width 0.5) (layer "F.Cu") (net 1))
 (segment (start 164.8 122.369304) (end 164.169304 123) (width 0.5) (layer "F.Cu") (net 1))
 (segment (start 159.200001 120.000001) (end 159.45 120.000001) (width 0.5) (layer "F.Cu") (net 1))
 (segment (start 171.025 114.526328) (end 169.898672 113.4) (width 1) (layer "F.Cu") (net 1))
 (via (at 165.4 117.649056) (size 0.8) (drill 0.4) (layers "F.Cu" "B.Cu") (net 1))
 (via (at 165.8 119.8) (size 0.8) (drill 0.4) (layers "F.Cu" "B.Cu") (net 1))
 (segment (start 165.4 117.649056) (end 165.4 119.4) (width 0.5) (layer "B.Cu") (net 1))
 (segment (start 165.4 119.4) (end 165.8 119.8) (width 0.5) (layer "B.Cu") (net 1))
 (segment (start 164.261997 117.861997) (end 163.4 117) (width 0.5) (layer "F.Cu") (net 5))
 (segment (start 160.45 117) (end 159.45 118) (width 0.5) (layer "F.Cu") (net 5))
 (segment (start 165.897708 121.321717) (end 166.480991 121.905) (width 0.5) (layer "F.Cu") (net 5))
 (segment (start 164.261997 118.29791) (end 164.261997 117.861997) (width 0.5) (layer "F.Cu") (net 5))
 (segment (start 166.480991 121.905) (end 167.625 121.905) (width 0.5) (layer "F.Cu") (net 5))
 (segment (start 163.4 117) (end 160.45 117) (width 0.5) (layer "F.Cu") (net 5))
 (via (at 164.261997 118.29791) (size 0.8) (drill 0.4) (layers "F.Cu" "B.Cu") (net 5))
 (via (at 165.897708 121.321717) (size 0.8) (drill 0.4) (layers "F.Cu" "B.Cu") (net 5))
 (segment (start 164.261997 119.686006) (end 165.897708 121.321717) (width 0.5) (layer "B.Cu") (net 5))
 (segment (start 164.261997 118.29791) (end 164.261997 119.686006) (width 0.5) (layer "B.Cu") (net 5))
 (segment (start 166.765 118.095) (end 167.625 118.095) (width 0.5) (layer "F.Cu") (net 10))
 (segment (start 163.84 121.96) (end 163.84 120.16) (width 0.5) (layer "F.Cu") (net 10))
 (segment (start 165.312 118.688) (end 166.172 118.688) (width 0.5) (layer "F.Cu") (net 10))
 (segment (start 163.84 120.16) (end 165.312 118.688) (width 0.5) (layer "F.Cu") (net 10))
 (segment (start 166.172 118.688) (end 166.765 118.095) (width 0.5) (layer "F.Cu") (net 10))
 (via (at 163.84 121.96) (size 0.8) (drill 0.4) (layers "F.Cu" "B.Cu") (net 10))
 (segment (start 163.84 121.96) (end 162.86 121.96) (width 0.5) (layer "B.Cu") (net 10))
 (segment (start 162.28 118) (end 162.375 118.095) (width 0.5) (layer "F.Cu") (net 6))
 (segment (start 161.2 118) (end 162.28 118) (width 0.5) (layer "F.Cu") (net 6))
 (via (at 161.2 118) (size 0.8) (drill 0.4) (layers "F.Cu" "B.Cu") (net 6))
 (segment (start 162.86 118) (end 161.2 118) (width 0.5) (layer "B.Cu") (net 6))
 (segment (start 161.2 119.4) (end 162.34 119.4) (width 0.5) (layer "F.Cu") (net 7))
 (segment (start 162.34 119.4) (end 162.375 119.365) (width 0.5) (layer "F.Cu") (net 7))
 (via (at 161.2 119.4) (size 0.8) (drill 0.4) (layers "F.Cu" "B.Cu") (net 7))
 (segment (start 161.2 119.4) (end 162.78 119.4) (width 0.5) (layer "B.Cu") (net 7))
 (segment (start 162.78 119.4) (end 162.86 119.32) (width 0.5) (layer "B.Cu") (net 7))
 (segment (start 161.2 120.6) (end 162.34 120.6) (width 0.5) (layer "F.Cu") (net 8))
 (segment (start 162.34 120.6) (end 162.375 120.635) (width 0.5) (layer "F.Cu") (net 8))
 (via (at 161.2 120.6) (size 0.8) (drill 0.4) (layers "F.Cu" "B.Cu") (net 8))
 (segment (start 161.2 120.6) (end 162.82 120.6) (width 0.5) (layer "B.Cu") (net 8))
 (segment (start 162.82 120.6) (end 162.86 120.64) (width 0.5) (layer "B.Cu") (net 8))
 (segment (start 169.375 114.8) (end 168.8 114.8) (width 0.5) (layer "F.Cu") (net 3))
 (via (at 168.8 114.8) (size 0.8) (drill 0.4) (layers "F.Cu" "B.Cu") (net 3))
 (segment (start 168.24 119.36) (end 168.8 118.8) (width 0.5) (layer "B.Cu") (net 3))
 (segment (start 168.8 118.8) (end 168.8 114.8) (width 0.5) (layer "B.Cu") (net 3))
 (segment (start 167.14 119.36) (end 168.24 119.36) (width 0.5) (layer "B.Cu") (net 3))
 (segment (start 161.2 125.2) (end 160.625 125.2) (width 0.5) (layer "F.Cu") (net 11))
 (via (at 161.2 125.2) (size 0.8) (drill 0.4) (layers "F.Cu" "B.Cu") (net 11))
 (segment (start 167 122) (end 166 123) (width 0.5) (layer "B.Cu") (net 11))
 (segment (start 166 123) (end 163.4 123) (width 0.5) (layer "B.Cu") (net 11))
 (segment (start 163.4 123) (end 161.2 125.2) (width 0.5) (layer "B.Cu") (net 11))
 (segment (start 167.14 122) (end 167 122) (width 0.5) (layer "B.Cu") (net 11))
 (segment (start 169.375 125.175) (end 168.8 124.6) (width 0.5) (layer "F.Cu") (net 2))
 (segment (start 169.375 125.2) (end 169.375 125.175) (width 0.5) (layer "F.Cu") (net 2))
 (via (at 168.8 124.6) (size 0.8) (drill 0.4) (layers "F.Cu" "B.Cu") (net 2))
 (segment (start 167.14 120.68) (end 168.08 120.68) (width 0.5) (layer "B.Cu") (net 2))
 (segment (start 168.08 120.68) (end 168.8 121.4) (width 0.5) (layer "B.Cu") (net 2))
 (segment (start 168.8 121.4) (end 168.8 124.6) (width 0.5) (layer "B.Cu") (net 2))
 (segment (start 160.625 114.8) (end 160.625 114.825) (width 0.5) (layer "F.Cu") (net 13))
 (segment (start 160.625 114.825) (end 161.2 115.4) (width 0.5) (layer "F.Cu") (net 13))
 (via (at 161.2 115.4) (size 0.8) (drill 0.4) (layers "F.Cu" "B.Cu") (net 13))
 (segment (start 166.098948 116.698948) (end 162.498948 116.698948) (width 0.5) (layer "B.Cu") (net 13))
 (segment (start 167.14 118.04) (end 167.14 117.74) (width 0.5) (layer "B.Cu") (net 13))
 (segment (start 162.498948 116.698948) (end 161.2 115.4) (width 0.5) (layer "B.Cu") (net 13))
 (segment (start 167.14 117.74) (end 166.098948 116.698948) (width 0.5) (layer "B.Cu") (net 13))
 (segment (start 168.365 120.635) (end 169 120) (width 0.5) (layer "F.Cu") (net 9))
 (segment (start 169 120) (end 169 117.6) (width 0.5) (layer "F.Cu") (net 9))
 (segment (start 169 117.6) (end 168.2 116.8) (width 0.5) (layer "F.Cu") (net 9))
 (segment (start 167.625 120.635) (end 168.365 120.635) (width 0.5) (layer "F.Cu") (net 9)))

